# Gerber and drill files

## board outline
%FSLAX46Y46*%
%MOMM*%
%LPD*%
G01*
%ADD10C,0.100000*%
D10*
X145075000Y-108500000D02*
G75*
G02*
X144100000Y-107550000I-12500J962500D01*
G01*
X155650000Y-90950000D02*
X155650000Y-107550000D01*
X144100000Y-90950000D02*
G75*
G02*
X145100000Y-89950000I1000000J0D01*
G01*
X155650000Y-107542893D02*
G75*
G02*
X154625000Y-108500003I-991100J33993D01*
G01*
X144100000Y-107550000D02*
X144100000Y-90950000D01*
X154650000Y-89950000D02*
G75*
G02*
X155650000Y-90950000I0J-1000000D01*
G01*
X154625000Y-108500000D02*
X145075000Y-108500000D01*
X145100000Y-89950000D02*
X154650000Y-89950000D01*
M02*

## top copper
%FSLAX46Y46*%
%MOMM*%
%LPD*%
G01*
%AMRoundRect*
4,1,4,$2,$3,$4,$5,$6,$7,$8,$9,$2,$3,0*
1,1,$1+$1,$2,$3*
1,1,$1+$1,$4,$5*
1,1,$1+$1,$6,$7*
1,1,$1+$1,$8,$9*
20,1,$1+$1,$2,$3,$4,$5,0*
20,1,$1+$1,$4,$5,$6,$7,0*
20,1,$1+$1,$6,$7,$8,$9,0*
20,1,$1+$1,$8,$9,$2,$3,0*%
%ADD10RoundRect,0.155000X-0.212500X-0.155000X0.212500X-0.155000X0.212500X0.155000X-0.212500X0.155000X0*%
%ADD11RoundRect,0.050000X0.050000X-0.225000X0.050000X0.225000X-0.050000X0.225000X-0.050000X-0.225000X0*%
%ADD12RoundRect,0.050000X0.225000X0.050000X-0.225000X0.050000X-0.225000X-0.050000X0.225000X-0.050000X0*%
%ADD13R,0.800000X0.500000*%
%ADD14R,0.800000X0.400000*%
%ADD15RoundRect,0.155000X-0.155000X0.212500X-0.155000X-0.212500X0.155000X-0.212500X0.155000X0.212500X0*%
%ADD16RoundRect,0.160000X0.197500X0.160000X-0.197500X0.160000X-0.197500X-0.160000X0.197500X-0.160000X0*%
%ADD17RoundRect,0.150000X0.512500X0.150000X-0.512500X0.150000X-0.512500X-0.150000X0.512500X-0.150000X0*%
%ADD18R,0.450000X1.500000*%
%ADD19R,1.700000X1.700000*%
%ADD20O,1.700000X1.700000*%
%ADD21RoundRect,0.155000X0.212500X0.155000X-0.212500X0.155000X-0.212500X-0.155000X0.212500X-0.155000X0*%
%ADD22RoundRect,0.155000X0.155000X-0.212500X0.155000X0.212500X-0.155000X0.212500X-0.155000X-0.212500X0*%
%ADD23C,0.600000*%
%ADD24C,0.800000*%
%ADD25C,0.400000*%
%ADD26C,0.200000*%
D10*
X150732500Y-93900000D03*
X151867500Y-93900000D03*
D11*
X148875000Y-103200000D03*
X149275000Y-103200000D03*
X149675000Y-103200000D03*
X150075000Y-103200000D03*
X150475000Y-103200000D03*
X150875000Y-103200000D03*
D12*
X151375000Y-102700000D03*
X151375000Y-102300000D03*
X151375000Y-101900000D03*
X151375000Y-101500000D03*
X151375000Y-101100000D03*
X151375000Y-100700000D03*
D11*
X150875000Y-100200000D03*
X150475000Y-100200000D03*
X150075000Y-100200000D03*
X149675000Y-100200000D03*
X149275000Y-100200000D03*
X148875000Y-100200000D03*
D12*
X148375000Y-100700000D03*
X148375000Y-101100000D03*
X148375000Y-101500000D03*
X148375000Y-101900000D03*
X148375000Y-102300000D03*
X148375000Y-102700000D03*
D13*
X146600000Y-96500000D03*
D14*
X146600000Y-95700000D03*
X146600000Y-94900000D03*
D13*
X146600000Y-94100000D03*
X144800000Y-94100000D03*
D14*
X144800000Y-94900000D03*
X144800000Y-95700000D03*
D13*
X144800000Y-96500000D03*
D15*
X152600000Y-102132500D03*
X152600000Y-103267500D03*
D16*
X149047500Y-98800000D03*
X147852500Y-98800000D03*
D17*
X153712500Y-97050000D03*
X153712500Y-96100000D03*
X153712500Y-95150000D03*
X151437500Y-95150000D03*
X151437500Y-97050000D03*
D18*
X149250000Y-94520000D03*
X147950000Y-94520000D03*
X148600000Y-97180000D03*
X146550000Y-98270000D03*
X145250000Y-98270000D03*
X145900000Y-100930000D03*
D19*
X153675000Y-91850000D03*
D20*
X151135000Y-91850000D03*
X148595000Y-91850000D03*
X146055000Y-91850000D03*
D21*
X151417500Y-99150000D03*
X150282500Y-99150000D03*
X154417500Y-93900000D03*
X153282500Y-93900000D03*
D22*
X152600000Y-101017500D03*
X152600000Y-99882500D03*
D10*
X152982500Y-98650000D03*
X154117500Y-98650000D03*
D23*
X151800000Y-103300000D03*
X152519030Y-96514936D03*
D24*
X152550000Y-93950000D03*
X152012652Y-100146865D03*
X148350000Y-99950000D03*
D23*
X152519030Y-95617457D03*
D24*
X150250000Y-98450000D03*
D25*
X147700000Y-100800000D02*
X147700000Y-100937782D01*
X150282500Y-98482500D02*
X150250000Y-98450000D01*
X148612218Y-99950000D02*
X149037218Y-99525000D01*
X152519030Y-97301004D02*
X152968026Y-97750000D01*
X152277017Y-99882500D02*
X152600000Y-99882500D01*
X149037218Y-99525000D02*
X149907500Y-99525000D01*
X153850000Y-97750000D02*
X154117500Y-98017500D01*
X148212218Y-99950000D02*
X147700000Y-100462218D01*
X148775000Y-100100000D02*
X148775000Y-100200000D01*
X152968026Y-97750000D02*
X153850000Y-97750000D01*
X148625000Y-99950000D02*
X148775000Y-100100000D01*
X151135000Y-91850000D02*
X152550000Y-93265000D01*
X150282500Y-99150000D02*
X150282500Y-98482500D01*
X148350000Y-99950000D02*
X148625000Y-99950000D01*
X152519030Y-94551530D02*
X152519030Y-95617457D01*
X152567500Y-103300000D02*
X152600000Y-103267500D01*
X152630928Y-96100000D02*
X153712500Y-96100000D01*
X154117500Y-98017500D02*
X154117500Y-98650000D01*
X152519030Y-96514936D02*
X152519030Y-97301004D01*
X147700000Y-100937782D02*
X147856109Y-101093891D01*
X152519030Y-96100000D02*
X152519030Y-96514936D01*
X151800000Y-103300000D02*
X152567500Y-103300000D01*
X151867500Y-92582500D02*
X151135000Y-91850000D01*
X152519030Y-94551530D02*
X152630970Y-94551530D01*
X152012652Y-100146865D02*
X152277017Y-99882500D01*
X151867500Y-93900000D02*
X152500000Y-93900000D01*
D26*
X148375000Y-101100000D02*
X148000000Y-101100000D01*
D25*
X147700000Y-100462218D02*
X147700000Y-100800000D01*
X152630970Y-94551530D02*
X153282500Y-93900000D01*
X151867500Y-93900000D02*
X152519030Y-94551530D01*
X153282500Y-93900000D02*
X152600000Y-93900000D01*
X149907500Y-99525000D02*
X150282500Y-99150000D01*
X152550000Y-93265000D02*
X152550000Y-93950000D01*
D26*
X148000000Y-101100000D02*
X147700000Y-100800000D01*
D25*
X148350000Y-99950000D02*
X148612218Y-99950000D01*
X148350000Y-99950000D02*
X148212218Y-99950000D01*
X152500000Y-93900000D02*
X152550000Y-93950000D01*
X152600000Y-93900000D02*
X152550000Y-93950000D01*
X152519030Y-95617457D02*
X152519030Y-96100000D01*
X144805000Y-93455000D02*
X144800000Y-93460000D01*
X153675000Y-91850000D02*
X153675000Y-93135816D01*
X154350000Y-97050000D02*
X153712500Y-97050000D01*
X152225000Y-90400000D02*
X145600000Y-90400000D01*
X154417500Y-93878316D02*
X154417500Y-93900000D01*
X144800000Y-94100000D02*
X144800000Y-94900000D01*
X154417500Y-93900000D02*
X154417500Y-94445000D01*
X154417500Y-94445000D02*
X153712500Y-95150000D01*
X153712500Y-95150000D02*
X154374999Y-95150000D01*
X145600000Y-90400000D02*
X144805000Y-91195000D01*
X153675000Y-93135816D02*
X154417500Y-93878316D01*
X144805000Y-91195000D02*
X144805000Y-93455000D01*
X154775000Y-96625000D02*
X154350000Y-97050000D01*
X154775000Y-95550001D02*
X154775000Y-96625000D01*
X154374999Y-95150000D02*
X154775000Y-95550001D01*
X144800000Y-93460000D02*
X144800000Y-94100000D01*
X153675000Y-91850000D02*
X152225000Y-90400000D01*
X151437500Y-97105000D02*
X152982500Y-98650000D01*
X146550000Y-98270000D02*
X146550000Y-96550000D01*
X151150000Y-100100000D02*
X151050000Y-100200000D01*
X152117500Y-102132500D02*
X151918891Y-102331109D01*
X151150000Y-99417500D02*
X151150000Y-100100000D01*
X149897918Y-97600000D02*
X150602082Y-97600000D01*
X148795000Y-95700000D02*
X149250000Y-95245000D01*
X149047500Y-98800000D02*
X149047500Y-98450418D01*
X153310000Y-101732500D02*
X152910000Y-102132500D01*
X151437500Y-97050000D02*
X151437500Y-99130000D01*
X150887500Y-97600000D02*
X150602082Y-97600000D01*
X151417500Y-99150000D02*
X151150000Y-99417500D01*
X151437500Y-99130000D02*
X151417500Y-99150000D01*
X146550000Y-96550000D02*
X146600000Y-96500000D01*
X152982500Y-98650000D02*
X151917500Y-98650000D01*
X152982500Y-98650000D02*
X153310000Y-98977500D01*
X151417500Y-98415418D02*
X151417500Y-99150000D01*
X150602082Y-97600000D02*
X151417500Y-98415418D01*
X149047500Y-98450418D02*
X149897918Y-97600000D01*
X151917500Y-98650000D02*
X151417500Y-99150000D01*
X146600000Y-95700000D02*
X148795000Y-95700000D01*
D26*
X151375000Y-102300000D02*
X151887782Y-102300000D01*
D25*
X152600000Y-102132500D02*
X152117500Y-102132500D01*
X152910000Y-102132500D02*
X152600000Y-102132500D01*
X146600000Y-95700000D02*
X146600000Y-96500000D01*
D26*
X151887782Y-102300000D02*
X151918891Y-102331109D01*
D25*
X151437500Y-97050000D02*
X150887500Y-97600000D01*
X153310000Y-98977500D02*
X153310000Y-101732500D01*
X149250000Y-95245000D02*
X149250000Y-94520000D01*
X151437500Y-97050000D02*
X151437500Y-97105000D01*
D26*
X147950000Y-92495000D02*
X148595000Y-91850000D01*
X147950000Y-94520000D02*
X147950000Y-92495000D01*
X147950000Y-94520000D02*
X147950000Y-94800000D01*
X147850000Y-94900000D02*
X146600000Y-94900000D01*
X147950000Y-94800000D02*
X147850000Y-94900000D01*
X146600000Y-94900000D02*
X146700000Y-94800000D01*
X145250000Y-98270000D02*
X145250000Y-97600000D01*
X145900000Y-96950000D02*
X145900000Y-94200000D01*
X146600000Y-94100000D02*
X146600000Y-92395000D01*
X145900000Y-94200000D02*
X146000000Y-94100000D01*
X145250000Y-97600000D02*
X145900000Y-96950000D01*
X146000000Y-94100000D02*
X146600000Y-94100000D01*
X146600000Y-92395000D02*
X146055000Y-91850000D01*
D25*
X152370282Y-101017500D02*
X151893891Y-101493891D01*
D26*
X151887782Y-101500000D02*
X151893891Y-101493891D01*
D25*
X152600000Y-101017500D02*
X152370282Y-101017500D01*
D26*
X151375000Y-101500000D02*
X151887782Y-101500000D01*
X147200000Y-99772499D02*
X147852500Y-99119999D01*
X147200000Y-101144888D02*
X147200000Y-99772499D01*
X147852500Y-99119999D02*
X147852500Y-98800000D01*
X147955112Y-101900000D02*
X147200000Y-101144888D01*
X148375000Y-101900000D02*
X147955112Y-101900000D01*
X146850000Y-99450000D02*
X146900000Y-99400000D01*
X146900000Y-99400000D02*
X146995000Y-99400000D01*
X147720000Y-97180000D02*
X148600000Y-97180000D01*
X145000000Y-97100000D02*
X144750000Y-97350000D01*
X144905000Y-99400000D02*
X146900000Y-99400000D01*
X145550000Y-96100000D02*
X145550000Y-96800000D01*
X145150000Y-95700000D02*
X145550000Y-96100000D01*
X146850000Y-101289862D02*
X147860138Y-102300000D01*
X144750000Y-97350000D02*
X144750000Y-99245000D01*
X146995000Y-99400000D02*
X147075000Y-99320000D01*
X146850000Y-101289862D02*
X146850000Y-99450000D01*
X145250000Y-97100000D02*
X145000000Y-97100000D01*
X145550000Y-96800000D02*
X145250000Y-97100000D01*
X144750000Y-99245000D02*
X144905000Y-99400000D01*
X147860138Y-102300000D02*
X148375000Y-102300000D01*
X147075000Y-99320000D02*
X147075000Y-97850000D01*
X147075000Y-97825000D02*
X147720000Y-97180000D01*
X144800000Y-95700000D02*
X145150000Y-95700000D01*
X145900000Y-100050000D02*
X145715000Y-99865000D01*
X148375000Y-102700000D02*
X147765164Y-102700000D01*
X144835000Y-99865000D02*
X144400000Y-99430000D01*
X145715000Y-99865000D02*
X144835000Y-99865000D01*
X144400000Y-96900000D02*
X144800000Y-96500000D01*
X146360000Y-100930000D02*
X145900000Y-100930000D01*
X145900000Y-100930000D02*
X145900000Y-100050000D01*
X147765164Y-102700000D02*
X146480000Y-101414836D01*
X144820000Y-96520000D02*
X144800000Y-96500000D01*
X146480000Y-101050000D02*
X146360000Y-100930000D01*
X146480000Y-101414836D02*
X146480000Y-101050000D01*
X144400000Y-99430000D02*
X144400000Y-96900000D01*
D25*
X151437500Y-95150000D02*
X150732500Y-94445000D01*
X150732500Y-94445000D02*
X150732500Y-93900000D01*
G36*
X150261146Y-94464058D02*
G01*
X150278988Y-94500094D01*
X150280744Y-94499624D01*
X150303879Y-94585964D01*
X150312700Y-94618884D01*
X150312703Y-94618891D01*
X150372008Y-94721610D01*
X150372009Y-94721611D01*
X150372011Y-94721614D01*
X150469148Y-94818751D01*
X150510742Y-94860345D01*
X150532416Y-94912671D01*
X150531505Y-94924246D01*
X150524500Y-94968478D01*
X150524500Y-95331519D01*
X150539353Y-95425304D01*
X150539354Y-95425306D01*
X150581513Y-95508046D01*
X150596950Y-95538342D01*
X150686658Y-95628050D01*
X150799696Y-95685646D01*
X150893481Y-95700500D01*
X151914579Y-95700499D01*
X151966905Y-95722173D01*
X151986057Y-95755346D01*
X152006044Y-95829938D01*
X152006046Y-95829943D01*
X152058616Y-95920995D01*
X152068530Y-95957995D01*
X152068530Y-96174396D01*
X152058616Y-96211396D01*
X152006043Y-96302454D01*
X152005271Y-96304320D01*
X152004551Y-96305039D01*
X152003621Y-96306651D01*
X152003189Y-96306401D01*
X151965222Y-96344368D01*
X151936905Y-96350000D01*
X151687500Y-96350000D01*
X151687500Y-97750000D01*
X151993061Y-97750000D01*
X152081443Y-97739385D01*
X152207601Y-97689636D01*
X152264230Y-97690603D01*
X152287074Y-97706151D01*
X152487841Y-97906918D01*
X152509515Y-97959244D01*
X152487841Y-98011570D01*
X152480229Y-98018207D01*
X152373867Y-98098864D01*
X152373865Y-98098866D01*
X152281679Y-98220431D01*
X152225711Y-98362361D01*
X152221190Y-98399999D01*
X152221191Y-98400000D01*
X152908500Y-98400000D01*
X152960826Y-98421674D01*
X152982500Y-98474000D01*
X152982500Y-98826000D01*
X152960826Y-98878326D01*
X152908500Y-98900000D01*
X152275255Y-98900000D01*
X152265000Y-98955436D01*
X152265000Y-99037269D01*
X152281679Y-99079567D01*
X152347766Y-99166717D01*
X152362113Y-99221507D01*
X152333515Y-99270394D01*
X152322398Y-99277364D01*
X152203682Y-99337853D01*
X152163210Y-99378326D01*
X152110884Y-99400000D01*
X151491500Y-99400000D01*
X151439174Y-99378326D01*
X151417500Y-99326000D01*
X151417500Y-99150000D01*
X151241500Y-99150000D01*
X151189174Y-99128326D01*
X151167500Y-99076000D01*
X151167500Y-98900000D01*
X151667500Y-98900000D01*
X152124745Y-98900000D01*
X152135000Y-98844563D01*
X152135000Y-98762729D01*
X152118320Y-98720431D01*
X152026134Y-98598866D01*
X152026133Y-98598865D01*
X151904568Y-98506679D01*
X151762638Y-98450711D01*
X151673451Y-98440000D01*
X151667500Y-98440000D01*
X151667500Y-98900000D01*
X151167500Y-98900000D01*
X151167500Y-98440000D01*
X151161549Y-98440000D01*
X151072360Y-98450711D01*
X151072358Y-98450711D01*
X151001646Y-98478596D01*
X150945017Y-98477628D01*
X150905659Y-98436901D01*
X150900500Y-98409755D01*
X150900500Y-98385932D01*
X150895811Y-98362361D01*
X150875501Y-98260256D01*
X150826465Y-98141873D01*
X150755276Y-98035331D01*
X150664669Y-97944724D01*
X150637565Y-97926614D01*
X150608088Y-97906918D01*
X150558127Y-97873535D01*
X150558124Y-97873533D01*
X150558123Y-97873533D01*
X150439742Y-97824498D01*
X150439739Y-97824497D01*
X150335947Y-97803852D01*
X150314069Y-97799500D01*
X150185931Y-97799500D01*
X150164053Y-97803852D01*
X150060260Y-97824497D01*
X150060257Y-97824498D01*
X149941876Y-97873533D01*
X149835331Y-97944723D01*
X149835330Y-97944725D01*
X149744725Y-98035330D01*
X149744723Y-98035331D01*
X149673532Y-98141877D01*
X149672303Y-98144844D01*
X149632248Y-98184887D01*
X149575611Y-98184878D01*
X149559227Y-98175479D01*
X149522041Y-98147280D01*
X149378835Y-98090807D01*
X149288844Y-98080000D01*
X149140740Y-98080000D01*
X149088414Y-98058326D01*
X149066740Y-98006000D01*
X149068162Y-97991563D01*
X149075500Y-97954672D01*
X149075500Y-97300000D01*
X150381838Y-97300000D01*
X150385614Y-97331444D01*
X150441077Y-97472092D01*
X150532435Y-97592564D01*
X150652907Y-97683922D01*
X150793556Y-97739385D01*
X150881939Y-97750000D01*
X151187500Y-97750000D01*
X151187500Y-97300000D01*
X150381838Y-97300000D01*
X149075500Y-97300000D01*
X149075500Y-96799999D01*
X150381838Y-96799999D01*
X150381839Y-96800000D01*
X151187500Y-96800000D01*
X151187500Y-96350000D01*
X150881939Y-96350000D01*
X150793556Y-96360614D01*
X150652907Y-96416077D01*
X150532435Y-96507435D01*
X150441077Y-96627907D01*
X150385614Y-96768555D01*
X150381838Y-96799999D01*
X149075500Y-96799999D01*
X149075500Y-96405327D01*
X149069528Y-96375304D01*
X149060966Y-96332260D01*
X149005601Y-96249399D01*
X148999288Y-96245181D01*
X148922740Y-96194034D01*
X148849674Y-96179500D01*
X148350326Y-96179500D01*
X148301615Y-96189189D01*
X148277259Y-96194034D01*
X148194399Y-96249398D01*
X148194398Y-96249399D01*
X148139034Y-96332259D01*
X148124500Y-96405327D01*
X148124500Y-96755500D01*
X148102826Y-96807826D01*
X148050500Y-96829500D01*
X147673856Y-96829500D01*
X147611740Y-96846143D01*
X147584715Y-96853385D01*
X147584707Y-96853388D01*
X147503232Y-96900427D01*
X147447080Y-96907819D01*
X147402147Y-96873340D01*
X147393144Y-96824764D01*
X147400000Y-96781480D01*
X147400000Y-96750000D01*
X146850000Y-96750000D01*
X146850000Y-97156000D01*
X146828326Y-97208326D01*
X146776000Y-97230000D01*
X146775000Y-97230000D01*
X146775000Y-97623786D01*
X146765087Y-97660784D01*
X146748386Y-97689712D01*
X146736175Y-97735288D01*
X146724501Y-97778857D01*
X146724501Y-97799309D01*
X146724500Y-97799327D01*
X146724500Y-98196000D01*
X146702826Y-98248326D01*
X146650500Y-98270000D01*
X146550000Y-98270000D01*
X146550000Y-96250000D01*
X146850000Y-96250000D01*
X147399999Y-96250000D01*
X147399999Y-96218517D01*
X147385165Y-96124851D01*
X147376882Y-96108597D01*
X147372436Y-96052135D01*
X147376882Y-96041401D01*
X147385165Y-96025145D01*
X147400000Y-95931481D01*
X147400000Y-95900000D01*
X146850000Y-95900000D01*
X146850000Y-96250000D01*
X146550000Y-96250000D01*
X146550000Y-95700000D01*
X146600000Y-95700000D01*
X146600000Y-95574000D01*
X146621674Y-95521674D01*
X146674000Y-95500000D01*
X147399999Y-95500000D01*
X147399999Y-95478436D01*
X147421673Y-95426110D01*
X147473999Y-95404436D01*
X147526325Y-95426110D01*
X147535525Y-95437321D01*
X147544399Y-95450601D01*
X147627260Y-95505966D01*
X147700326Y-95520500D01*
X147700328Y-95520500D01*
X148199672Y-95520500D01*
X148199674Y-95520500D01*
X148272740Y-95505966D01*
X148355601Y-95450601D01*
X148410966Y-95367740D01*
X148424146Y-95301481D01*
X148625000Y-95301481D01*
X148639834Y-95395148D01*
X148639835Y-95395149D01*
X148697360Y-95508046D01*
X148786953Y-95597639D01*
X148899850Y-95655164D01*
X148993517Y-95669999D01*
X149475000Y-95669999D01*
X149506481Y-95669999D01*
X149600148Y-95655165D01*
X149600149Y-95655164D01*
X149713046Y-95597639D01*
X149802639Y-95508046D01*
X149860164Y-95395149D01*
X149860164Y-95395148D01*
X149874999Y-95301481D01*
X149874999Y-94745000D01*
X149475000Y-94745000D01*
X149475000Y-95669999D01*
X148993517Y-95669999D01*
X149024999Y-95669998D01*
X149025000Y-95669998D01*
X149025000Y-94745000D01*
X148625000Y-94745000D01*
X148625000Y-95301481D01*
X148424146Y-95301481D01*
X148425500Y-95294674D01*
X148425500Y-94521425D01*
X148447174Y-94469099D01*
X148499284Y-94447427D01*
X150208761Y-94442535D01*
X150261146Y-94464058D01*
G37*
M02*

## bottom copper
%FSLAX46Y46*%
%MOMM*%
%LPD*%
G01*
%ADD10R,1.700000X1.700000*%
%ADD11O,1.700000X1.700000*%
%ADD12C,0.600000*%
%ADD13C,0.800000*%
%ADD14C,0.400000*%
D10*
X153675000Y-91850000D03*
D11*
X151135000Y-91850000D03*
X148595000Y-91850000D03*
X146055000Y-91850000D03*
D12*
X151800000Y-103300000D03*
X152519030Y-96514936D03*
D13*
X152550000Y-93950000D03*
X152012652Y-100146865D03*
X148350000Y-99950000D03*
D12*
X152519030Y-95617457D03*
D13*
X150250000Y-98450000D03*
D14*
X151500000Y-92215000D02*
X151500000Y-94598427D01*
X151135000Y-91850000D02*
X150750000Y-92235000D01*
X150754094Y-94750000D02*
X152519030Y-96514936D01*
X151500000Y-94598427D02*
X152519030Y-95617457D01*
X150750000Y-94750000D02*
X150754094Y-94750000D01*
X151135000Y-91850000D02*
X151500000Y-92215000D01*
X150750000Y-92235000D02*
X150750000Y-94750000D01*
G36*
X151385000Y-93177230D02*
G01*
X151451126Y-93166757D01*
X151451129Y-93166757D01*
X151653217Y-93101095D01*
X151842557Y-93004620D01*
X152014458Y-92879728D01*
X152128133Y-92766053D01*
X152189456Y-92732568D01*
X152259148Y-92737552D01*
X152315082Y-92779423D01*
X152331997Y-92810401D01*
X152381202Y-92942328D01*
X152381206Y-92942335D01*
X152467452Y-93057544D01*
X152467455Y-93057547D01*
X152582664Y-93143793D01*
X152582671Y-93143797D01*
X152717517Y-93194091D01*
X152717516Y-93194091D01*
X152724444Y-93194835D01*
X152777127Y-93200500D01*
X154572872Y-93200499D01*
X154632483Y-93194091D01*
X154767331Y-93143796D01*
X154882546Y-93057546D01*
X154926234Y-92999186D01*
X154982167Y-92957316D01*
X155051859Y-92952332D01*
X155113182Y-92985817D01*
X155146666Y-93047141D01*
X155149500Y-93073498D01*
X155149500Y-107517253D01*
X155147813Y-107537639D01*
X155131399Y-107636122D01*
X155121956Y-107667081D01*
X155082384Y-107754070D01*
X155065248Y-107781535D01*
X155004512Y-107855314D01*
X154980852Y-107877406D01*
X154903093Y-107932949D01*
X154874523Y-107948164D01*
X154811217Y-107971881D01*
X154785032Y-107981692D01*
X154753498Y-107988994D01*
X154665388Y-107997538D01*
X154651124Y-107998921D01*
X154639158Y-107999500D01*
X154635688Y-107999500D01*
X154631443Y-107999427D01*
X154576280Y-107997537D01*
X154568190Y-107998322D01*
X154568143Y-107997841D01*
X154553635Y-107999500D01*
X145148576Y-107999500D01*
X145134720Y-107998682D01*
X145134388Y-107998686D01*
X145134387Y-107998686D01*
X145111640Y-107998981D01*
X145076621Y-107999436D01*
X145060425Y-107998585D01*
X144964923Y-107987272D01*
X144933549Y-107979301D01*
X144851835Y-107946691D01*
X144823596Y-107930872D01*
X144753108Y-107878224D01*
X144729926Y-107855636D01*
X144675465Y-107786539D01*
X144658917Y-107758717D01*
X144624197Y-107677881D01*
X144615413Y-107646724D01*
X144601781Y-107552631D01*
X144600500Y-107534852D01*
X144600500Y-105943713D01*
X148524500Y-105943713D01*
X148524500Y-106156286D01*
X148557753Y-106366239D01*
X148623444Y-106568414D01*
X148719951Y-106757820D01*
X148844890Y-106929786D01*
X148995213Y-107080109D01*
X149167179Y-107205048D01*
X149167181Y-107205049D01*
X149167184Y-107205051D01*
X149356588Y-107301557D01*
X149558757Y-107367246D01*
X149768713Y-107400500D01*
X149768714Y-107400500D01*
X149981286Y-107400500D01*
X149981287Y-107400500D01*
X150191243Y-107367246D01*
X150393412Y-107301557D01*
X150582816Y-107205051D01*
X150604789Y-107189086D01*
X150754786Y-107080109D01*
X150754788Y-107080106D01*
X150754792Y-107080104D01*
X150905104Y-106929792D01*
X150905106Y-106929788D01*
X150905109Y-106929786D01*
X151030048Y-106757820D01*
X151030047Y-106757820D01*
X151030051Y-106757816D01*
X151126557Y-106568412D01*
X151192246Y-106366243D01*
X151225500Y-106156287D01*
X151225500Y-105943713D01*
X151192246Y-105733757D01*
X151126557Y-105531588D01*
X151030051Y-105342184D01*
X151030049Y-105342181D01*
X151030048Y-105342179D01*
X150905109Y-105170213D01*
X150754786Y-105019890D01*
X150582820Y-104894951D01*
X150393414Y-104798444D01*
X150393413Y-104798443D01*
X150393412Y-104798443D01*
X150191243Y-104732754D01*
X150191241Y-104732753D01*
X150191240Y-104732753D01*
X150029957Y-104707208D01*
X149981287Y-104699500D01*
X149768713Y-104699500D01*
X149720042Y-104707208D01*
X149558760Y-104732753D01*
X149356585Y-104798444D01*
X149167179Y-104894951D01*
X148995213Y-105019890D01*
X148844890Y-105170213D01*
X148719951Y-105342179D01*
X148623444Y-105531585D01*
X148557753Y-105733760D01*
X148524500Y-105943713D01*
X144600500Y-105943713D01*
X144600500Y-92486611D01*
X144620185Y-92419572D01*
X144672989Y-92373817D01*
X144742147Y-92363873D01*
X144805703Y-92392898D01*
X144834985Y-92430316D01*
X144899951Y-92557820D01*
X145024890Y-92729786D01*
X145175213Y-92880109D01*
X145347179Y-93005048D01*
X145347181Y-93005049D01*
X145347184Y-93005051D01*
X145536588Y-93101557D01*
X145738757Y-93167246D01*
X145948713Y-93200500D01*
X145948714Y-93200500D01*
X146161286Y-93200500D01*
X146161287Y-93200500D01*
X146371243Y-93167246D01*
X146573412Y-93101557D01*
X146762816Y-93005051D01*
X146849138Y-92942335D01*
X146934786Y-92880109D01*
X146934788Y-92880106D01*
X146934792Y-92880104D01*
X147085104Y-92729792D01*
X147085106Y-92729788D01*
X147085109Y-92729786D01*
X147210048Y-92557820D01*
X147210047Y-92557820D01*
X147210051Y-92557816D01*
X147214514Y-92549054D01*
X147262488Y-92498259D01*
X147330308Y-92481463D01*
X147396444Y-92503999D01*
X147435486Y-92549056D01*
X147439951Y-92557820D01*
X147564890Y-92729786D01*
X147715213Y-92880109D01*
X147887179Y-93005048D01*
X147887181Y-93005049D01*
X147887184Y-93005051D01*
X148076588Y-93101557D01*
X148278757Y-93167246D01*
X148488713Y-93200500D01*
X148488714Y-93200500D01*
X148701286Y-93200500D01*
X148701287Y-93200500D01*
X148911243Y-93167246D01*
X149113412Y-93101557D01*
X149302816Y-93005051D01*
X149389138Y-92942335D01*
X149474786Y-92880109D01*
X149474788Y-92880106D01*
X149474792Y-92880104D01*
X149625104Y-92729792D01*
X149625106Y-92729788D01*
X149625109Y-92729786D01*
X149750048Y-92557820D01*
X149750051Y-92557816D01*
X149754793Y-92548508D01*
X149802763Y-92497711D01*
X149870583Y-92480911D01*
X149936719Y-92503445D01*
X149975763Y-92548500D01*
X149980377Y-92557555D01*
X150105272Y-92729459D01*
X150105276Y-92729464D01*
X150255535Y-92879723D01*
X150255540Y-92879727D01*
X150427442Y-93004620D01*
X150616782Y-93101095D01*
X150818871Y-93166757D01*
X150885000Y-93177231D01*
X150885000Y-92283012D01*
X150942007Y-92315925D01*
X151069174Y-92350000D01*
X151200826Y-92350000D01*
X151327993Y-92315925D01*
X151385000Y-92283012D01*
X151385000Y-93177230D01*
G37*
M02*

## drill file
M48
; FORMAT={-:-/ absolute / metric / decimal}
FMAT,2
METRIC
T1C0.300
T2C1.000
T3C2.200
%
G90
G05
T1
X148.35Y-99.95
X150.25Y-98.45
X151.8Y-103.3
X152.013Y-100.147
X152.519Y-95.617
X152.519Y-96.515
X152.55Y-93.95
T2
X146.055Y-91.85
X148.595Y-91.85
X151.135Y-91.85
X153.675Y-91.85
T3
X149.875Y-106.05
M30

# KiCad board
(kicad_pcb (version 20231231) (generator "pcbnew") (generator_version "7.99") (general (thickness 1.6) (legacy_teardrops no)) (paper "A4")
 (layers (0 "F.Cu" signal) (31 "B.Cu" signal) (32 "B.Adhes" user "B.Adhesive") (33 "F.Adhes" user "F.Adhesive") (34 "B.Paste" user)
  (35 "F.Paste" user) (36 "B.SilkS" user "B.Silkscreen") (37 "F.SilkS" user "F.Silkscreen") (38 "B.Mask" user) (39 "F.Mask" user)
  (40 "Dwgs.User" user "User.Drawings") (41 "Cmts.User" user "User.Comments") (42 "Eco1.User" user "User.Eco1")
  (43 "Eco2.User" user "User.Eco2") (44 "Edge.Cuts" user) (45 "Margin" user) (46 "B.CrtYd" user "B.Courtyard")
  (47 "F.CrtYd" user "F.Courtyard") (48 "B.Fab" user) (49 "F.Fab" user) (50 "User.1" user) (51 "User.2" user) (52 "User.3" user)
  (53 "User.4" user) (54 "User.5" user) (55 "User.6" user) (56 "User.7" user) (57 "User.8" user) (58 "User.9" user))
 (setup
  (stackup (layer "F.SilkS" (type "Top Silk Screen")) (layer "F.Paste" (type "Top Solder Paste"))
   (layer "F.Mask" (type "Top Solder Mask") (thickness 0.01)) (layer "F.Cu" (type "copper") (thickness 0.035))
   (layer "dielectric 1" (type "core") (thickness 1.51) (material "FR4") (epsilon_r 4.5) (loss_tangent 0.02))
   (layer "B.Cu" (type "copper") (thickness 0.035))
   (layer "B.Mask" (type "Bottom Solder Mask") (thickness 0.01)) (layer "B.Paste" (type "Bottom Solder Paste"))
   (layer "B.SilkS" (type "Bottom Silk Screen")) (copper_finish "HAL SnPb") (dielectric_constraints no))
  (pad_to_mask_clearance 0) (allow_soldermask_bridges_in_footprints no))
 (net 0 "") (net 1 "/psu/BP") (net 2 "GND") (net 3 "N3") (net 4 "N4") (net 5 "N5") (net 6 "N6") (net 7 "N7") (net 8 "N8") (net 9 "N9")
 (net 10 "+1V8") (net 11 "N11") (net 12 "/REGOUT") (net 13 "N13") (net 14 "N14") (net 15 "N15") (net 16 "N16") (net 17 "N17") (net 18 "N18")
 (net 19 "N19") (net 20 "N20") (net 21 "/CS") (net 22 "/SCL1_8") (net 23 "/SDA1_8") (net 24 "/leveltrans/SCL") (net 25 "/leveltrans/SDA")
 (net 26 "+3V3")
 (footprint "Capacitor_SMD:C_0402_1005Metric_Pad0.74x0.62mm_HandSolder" (layer "F.Cu") (at 151.3 93.9)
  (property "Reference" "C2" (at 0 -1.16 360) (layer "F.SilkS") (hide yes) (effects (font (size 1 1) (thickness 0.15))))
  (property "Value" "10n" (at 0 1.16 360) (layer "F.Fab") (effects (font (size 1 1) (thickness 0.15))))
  (pad "1" smd roundrect (at -0.5675 0) (size 0.735 0.62) (layers "F.Cu" "F.Paste" "F.Mask") (roundrect_rratio 0.25) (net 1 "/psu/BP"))
  (pad "2" smd roundrect (at 0.5675 0) (size 0.735 0.62) (layers "F.Cu" "F.Paste" "F.Mask") (roundrect_rratio 0.25) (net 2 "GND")))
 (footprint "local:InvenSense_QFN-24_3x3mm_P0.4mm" (layer "F.Cu") (at 149.875 101.7 90)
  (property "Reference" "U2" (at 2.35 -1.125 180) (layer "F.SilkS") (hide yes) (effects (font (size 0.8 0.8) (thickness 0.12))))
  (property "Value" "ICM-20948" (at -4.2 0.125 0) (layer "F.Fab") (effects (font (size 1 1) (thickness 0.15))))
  (pad "1" smd roundrect (at -1.5 -1 90) (size 0.55 0.2) (layers "F.Cu" "F.Paste" "F.Mask") (roundrect_rratio 0.25) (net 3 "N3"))
  (pad "2" smd roundrect (at -1.5 -0.6 90) (size 0.55 0.2) (layers "F.Cu" "F.Paste" "F.Mask") (roundrect_rratio 0.25) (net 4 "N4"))
  (pad "3" smd roundrect (at -1.5 -0.2 90) (size 0.55 0.2) (layers "F.Cu" "F.Paste" "F.Mask") (roundrect_rratio 0.25) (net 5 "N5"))
  (pad "4" smd roundrect (at -1.5 0.2 90) (size 0.55 0.2) (layers "F.Cu" "F.Paste" "F.Mask") (roundrect_rratio 0.25) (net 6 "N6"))
  (pad "5" smd roundrect (at -1.5 0.6 90) (size 0.55 0.2) (layers "F.Cu" "F.Paste" "F.Mask") (roundrect_rratio 0.25) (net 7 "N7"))
  (pad "6" smd roundrect (at -1.5 1 90) (size 0.55 0.2) (layers "F.Cu" "F.Paste" "F.Mask") (roundrect_rratio 0.25) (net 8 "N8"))
  (pad "7" smd roundrect (at -1 1.5 180) (size 0.55 0.2) (layers "F.Cu" "F.Paste" "F.Mask") (roundrect_rratio 0.25) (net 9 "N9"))
  (pad "8" smd roundrect (at -0.6 1.5 180) (size 0.55 0.2) (layers "F.Cu" "F.Paste" "F.Mask") (roundrect_rratio 0.25) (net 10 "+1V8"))
  (pad "9" smd roundrect (at -0.2 1.5 180) (size 0.55 0.2) (layers "F.Cu" "F.Paste" "F.Mask") (roundrect_rratio 0.25) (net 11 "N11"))
  (pad "10" smd roundrect (at 0.2 1.5 180) (size 0.55 0.2) (layers "F.Cu" "F.Paste" "F.Mask") (roundrect_rratio 0.25) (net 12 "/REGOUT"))
  (pad "11" smd roundrect (at 0.6 1.5 180) (size 0.55 0.2) (layers "F.Cu" "F.Paste" "F.Mask") (roundrect_rratio 0.25) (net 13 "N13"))
  (pad "12" smd roundrect (at 1 1.5 180) (size 0.55 0.2) (layers "F.Cu" "F.Paste" "F.Mask") (roundrect_rratio 0.25) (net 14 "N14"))
  (pad "13" smd roundrect (at 1.5 1 90) (size 0.55 0.2) (layers "F.Cu" "F.Paste" "F.Mask") (roundrect_rratio 0.25) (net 10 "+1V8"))
  (pad "14" smd roundrect (at 1.5 0.6 90) (size 0.55 0.2) (layers "F.Cu" "F.Paste" "F.Mask") (roundrect_rratio 0.25) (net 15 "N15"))
  (pad "15" smd roundrect (at 1.5 0.2 90) (size 0.55 0.2) (layers "F.Cu" "F.Paste" "F.Mask") (roundrect_rratio 0.25) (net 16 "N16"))
  (pad "16" smd roundrect (at 1.5 -0.2 90) (size 0.55 0.2) (layers "F.Cu" "F.Paste" "F.Mask") (roundrect_rratio 0.25) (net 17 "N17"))
  (pad "17" smd roundrect (at 1.5 -0.6 90) (size 0.55 0.2) (layers "F.Cu" "F.Paste" "F.Mask") (roundrect_rratio 0.25) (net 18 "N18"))
  (pad "18" smd roundrect (at 1.5 -1 90) (size 0.55 0.2) (layers "F.Cu" "F.Paste" "F.Mask") (roundrect_rratio 0.25) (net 2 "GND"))
  (pad "19" smd roundrect (at 1 -1.5 180) (size 0.55 0.2) (layers "F.Cu" "F.Paste" "F.Mask") (roundrect_rratio 0.25) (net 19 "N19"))
  (pad "20" smd roundrect (at 0.6 -1.5 180) (size 0.55 0.2) (layers "F.Cu" "F.Paste" "F.Mask") (roundrect_rratio 0.25) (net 2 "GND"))
  (pad "21" smd roundrect (at 0.2 -1.5 180) (size 0.55 0.2) (layers "F.Cu" "F.Paste" "F.Mask") (roundrect_rratio 0.25) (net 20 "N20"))
  (pad "22" smd roundrect (at -0.2 -1.5 180) (size 0.55 0.2) (layers "F.Cu" "F.Paste" "F.Mask") (roundrect_rratio 0.25) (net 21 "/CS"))
  (pad "23" smd roundrect (at -0.6 -1.5 180) (size 0.55 0.2) (layers "F.Cu" "F.Paste" "F.Mask") (roundrect_rratio 0.25) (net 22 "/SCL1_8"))
  (pad "24" smd roundrect (at -1 -1.5 180) (size 0.55 0.2) (layers "F.Cu" "F.Paste" "F.Mask") (roundrect_rratio 0.25) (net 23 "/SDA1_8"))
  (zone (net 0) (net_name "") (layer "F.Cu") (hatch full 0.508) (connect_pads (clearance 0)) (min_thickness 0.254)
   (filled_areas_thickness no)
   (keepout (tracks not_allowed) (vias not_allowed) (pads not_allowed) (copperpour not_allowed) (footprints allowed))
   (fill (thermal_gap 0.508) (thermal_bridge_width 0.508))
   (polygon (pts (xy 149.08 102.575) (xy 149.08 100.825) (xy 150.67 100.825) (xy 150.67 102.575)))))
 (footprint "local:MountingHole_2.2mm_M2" (layer "F.Cu") (at 149.875 106.05)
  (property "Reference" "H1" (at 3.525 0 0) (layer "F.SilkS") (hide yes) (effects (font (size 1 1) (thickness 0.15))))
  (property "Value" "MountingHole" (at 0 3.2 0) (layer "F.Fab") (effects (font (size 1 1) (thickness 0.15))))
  (pad "" np_thru_hole circle (at 0 0) (size 2.2 2.2) (drill 2.2) (layers "*.Cu" "*.Mask")))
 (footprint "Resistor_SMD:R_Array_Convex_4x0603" (layer "F.Cu") (at 145.7 95.3 180)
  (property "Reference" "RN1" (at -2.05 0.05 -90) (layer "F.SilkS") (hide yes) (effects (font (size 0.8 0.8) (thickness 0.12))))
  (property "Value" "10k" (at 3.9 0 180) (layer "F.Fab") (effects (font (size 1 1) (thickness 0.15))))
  (pad "1" smd rect (at -0.9 -1.2 180) (size 0.8 0.5) (layers "F.Cu" "F.Paste" "F.Mask") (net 10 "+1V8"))
  (pad "2" smd rect (at -0.9 -0.4 180) (size 0.8 0.4) (layers "F.Cu" "F.Paste" "F.Mask") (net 10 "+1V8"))
  (pad "3" smd rect (at -0.9 0.4 180) (size 0.8 0.4) (layers "F.Cu" "F.Paste" "F.Mask") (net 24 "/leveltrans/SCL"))
  (pad "4" smd rect (at -0.9 1.2 180) (size 0.8 0.5) (layers "F.Cu" "F.Paste" "F.Mask") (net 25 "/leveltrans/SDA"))
  (pad "5" smd rect (at 0.9 1.2 180) (size 0.8 0.5) (layers "F.Cu" "F.Paste" "F.Mask") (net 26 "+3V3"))
  (pad "6" smd rect (at 0.9 0.4 180) (size 0.8 0.4) (layers "F.Cu" "F.Paste" "F.Mask") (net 26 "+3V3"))
  (pad "7" smd rect (at 0.9 -0.4 180) (size 0.8 0.4) (layers "F.Cu" "F.Paste" "F.Mask") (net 22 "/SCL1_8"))
  (pad "8" smd rect (at 0.9 -1.2 180) (size 0.8 0.5) (layers "F.Cu" "F.Paste" "F.Mask") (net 23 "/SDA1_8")))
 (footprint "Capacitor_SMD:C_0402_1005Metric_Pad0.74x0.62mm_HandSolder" (layer "F.Cu") (at 152.6 102.7 -90)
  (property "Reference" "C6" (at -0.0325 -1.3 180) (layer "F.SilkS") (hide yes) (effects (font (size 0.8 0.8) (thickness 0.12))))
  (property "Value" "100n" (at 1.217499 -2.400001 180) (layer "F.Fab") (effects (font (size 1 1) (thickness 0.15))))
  (pad "1" smd roundrect (at -0.5675 0 270) (size 0.735 0.62) (layers "F.Cu" "F.Paste" "F.Mask") (roundrect_rratio 0.25) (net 10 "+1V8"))
  (pad "2" smd roundrect (at 0.5675 0 270) (size 0.735 0.62) (layers "F.Cu" "F.Paste" "F.Mask") (roundrect_rratio 0.25) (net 2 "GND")))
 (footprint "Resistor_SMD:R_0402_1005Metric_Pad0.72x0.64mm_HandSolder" (layer "F.Cu") (at 148.45 98.8 180)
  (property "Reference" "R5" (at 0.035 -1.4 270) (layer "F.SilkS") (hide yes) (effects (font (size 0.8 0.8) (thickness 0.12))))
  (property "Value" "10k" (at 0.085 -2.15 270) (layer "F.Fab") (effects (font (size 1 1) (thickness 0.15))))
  (pad "1" smd roundrect (at -0.5975 0 180) (size 0.715 0.64) (layers "F.Cu" "F.Paste" "F.Mask") (roundrect_rratio 0.25) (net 10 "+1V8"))
  (pad "2" smd roundrect (at 0.5975 0 180) (size 0.715 0.64) (layers "F.Cu" "F.Paste" "F.Mask") (roundrect_rratio 0.25) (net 21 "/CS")))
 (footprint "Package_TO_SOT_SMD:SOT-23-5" (layer "F.Cu") (at 152.575 96.1 180)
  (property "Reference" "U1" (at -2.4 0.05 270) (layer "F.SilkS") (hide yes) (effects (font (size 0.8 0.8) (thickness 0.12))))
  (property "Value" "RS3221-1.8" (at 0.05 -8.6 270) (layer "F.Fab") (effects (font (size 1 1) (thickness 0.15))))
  (pad "1" smd roundrect (at -1.1375 -0.95 180) (size 1.325 0.6) (layers "F.Cu" "F.Paste" "F.Mask") (roundrect_rratio 0.25) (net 26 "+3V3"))
  (pad "2" smd roundrect (at -1.1375 0 180) (size 1.325 0.6) (layers "F.Cu" "F.Paste" "F.Mask") (roundrect_rratio 0.25) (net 2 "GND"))
  (pad "3" smd roundrect (at -1.1375 0.95 180) (size 1.325 0.6) (layers "F.Cu" "F.Paste" "F.Mask") (roundrect_rratio 0.25) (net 26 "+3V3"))
  (pad "4" smd roundrect (at 1.1375 0.95 180) (size 1.325 0.6) (layers "F.Cu" "F.Paste" "F.Mask") (roundrect_rratio 0.25) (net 1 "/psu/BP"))
  (pad "5" smd roundrect (at 1.1375 -0.95 180) (size 1.325 0.6) (layers "F.Cu" "F.Paste" "F.Mask") (roundrect_rratio 0.25) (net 10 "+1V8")))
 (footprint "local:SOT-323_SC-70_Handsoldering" (layer "F.Cu") (at 148.6 95.85 -90)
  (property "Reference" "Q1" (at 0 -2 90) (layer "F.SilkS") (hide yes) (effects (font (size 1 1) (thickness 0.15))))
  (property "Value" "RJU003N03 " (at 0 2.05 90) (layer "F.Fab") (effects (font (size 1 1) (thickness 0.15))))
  (pad "1" smd rect (at -1.33 -0.65 180) (size 0.45 1.5) (layers "F.Cu" "F.Paste" "F.Mask") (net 10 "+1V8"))
  (pad "2" smd rect (at -1.33 0.65 180) (size 0.45 1.5) (layers "F.Cu" "F.Paste" "F.Mask") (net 24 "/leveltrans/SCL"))
  (pad "3" smd rect (at 1.33 0 180) (size 0.45 1.5) (layers "F.Cu" "F.Paste" "F.Mask") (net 22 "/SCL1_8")))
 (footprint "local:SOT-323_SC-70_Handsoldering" (layer "F.Cu") (at 145.9 99.6 -90)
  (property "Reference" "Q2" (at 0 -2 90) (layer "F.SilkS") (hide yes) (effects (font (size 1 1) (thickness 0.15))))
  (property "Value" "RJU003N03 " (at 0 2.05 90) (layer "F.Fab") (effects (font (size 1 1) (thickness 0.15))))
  (pad "1" smd rect (at -1.33 -0.65 180) (size 0.45 1.5) (layers "F.Cu" "F.Paste" "F.Mask") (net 10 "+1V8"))
  (pad "2" smd rect (at -1.33 0.65 180) (size 0.45 1.5) (layers "F.Cu" "F.Paste" "F.Mask") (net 25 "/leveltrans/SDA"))
  (pad "3" smd rect (at 1.33 0 180) (size 0.45 1.5) (layers "F.Cu" "F.Paste" "F.Mask") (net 23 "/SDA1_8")))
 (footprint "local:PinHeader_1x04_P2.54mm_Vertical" (layer "F.Cu") (at 153.675 91.85 -90)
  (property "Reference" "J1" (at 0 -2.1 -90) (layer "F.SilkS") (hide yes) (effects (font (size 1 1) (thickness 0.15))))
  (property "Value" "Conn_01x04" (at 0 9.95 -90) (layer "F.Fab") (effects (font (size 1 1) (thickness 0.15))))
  (pad "1" thru_hole rect (at 0 0 270) (size 1.7 1.7) (drill 1) (layers "*.Cu" "*.Mask") (remove_unused_layers no) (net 26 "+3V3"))
  (pad "2" thru_hole oval (at 0 2.54 270) (size 1.7 1.7) (drill 1) (layers "*.Cu" "*.Mask") (remove_unused_layers no) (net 2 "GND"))
  (pad "3" thru_hole oval (at 0 5.08 270) (size 1.7 1.7) (drill 1) (layers "*.Cu" "*.Mask") (remove_unused_layers no)
   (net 24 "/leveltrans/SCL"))
  (pad "4" thru_hole oval (at 0 7.62 270) (size 1.7 1.7) (drill 1) (layers "*.Cu" "*.Mask") (remove_unused_layers no)
   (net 25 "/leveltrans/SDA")))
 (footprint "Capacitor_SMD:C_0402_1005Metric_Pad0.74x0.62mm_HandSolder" (layer "F.Cu") (at 150.85 99.15 180)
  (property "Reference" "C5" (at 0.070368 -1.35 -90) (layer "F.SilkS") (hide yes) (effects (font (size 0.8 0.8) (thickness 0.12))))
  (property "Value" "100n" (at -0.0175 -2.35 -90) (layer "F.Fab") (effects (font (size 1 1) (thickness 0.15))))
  (pad "1" smd roundrect (at -0.5675 0 180) (size 0.735 0.62) (layers "F.Cu" "F.Paste" "F.Mask") (roundrect_rratio 0.25) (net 10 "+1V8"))
  (pad "2" smd roundrect (at 0.5675 0 180) (size 0.735 0.62) (layers "F.Cu" "F.Paste" "F.Mask") (roundrect_rratio 0.25) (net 2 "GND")))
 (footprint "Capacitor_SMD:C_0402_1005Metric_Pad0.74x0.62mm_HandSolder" (layer "F.Cu") (at 153.85 93.9 180)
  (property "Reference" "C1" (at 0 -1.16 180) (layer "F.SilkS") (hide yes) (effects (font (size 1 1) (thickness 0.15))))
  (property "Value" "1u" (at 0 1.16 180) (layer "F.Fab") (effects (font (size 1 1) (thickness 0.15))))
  (pad "1" smd roundrect (at -0.5675 0 180) (size 0.735 0.62) (layers "F.Cu" "F.Paste" "F.Mask") (roundrect_rratio 0.25) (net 26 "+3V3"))
  (pad "2" smd roundrect (at 0.5675 0 180) (size 0.735 0.62) (layers "F.Cu" "F.Paste" "F.Mask") (roundrect_rratio 0.25) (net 2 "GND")))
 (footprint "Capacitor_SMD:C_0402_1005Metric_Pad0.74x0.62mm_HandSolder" (layer "F.Cu") (at 152.6 100.45 90)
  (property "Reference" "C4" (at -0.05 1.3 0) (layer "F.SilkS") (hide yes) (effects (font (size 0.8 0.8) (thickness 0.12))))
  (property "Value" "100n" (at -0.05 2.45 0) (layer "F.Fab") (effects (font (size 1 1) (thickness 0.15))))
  (pad "1" smd roundrect (at -0.5675 0 90) (size 0.735 0.62) (layers "F.Cu" "F.Paste" "F.Mask") (roundrect_rratio 0.25) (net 12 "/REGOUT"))
  (pad "2" smd roundrect (at 0.5675 0 90) (size 0.735 0.62) (layers "F.Cu" "F.Paste" "F.Mask") (roundrect_rratio 0.25) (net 2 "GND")))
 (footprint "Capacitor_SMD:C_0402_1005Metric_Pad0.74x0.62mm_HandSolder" (layer "F.Cu") (at 153.55 98.65)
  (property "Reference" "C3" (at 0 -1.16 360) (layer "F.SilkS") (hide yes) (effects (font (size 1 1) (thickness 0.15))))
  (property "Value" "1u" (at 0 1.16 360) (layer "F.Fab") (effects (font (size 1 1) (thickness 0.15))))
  (pad "1" smd roundrect (at -0.5675 0) (size 0.735 0.62) (layers "F.Cu" "F.Paste" "F.Mask") (roundrect_rratio 0.25) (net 10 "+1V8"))
  (pad "2" smd roundrect (at 0.5675 0) (size 0.735 0.62) (layers "F.Cu" "F.Paste" "F.Mask") (roundrect_rratio 0.25) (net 2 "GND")))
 (gr_arc (start 145.075 108.5) (mid 144.390748 108.226929) (end 144.1 107.55) (stroke (width 0.1) (type default)) (layer "Edge.Cuts"))
 (gr_line (start 155.65 90.95) (end 155.65 107.55) (stroke (width 0.1) (type default)) (layer "Edge.Cuts"))
 (gr_arc (start 144.1 90.95) (mid 144.392893 90.242893) (end 145.1 89.95) (stroke (width 0.1) (type default)) (layer "Edge.Cuts"))
 (gr_arc (start 155.65 107.542893) (mid 155.335723 108.23373) (end 154.625 108.5) (stroke (width 0.1) (type default)) (layer "Edge.Cuts"))
 (gr_line (start 144.1 107.55) (end 144.1 90.95) (stroke (width 0.1) (type default)) (layer "Edge.Cuts"))
 (gr_arc (start 154.65 89.95) (mid 155.357107 90.242893) (end 155.65 90.95) (stroke (width 0.1) (type default)) (layer "Edge.Cuts"))
 (gr_line (start 154.625 108.5) (end 145.075 108.5) (stroke (width 0.1) (type default)) (layer "Edge.Cuts"))
 (gr_line (start 145.1 89.95) (end 154.65 89.95) (stroke (width 0.1) (type default)) (layer "Edge.Cuts"))
 (segment (start 147.7 100.8) (end 147.7 100.937782) (width 0.4) (layer "F.Cu") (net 2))
 (segment (start 150.2825 98.4825) (end 150.25 98.45) (width 0.4) (layer "F.Cu") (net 2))
 (segment (start 148.612218 99.95) (end 149.037218 99.525) (width 0.4) (layer "F.Cu") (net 2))
 (segment (start 152.51903 97.301004) (end 152.968026 97.75) (width 0.4) (layer "F.Cu") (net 2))
 (segment (start 152.277017 99.8825) (end 152.6 99.8825) (width 0.4) (layer "F.Cu") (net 2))
 (segment (start 149.037218 99.525) (end 149.9075 99.525) (width 0.4) (layer "F.Cu") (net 2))
 (segment (start 153.85 97.75) (end 154.1175 98.0175) (width 0.4) (layer "F.Cu") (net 2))
 (segment (start 148.212218 99.95) (end 147.7 100.462218) (width 0.4) (layer "F.Cu") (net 2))
 (segment (start 148.775 100.1) (end 148.775 100.2) (width 0.4) (layer "F.Cu") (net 2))
 (segment (start 152.968026 97.75) (end 153.85 97.75) (width 0.4) (layer "F.Cu") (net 2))
 (segment (start 148.625 99.95) (end 148.775 100.1) (width 0.4) (layer "F.Cu") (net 2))
 (segment (start 151.135 91.85) (end 152.55 93.265) (width 0.4) (layer "F.Cu") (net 2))
 (segment (start 150.2825 99.15) (end 150.2825 98.4825) (width 0.4) (layer "F.Cu") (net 2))
 (segment (start 148.35 99.95) (end 148.625 99.95) (width 0.4) (layer "F.Cu") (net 2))
 (segment (start 152.51903 94.55153) (end 152.51903 95.617457) (width 0.4) (layer "F.Cu") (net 2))
 (segment (start 152.5675 103.3) (end 152.6 103.2675) (width 0.4) (layer "F.Cu") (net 2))
 (segment (start 152.630928 96.1) (end 153.7125 96.1) (width 0.4) (layer "F.Cu") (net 2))
 (segment (start 154.1175 98.0175) (end 154.1175 98.65) (width 0.4) (layer "F.Cu") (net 2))
 (segment (start 152.51903 96.514936) (end 152.51903 97.301004) (width 0.4) (layer "F.Cu") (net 2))
 (segment (start 147.7 100.937782) (end 147.856109 101.093891) (width 0.4) (layer "F.Cu") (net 2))
 (segment (start 152.51903 96.1) (end 152.51903 96.514936) (width 0.4) (layer "F.Cu") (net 2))
 (segment (start 151.8 103.3) (end 152.5675 103.3) (width 0.4) (layer "F.Cu") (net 2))
 (segment (start 151.8675 92.5825) (end 151.135 91.85) (width 0.4) (layer "F.Cu") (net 2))
 (segment (start 152.51903 94.55153) (end 152.63097 94.55153) (width 0.4) (layer "F.Cu") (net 2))
 (segment (start 152.012652 100.146865) (end 152.277017 99.8825) (width 0.4) (layer "F.Cu") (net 2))
 (segment (start 151.8675 93.9) (end 152.5 93.9) (width 0.4) (layer "F.Cu") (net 2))
 (segment (start 148.375 101.1) (end 148 101.1) (width 0.2) (layer "F.Cu") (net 2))
 (segment (start 147.7 100.462218) (end 147.7 100.8) (width 0.4) (layer "F.Cu") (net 2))
 (segment (start 152.63097 94.55153) (end 153.2825 93.9) (width 0.4) (layer "F.Cu") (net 2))
 (segment (start 151.8675 93.9) (end 152.51903 94.55153) (width 0.4) (layer "F.Cu") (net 2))
 (segment (start 153.2825 93.9) (end 152.6 93.9) (width 0.4) (layer "F.Cu") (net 2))
 (segment (start 149.9075 99.525) (end 150.2825 99.15) (width 0.4) (layer "F.Cu") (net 2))
 (segment (start 152.55 93.265) (end 152.55 93.95) (width 0.4) (layer "F.Cu") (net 2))
 (segment (start 148 101.1) (end 147.7 100.8) (width 0.2) (layer "F.Cu") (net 2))
 (segment (start 148.35 99.95) (end 148.612218 99.95) (width 0.4) (layer "F.Cu") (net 2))
 (segment (start 148.35 99.95) (end 148.212218 99.95) (width 0.4) (layer "F.Cu") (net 2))
 (segment (start 152.5 93.9) (end 152.55 93.95) (width 0.4) (layer "F.Cu") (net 2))
 (segment (start 152.6 93.9) (end 152.55 93.95) (width 0.4) (layer "F.Cu") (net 2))
 (segment (start 152.51903 95.617457) (end 152.51903 96.1) (width 0.4) (layer "F.Cu") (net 2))
 (via (at 151.8 103.3) (size 0.6) (drill 0.3) (layers "F.Cu" "B.Cu") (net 2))
 (via (at 152.51903 96.514936) (size 0.6) (drill 0.3) (layers "F.Cu" "B.Cu") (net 2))
 (via (at 152.55 93.95) (size 0.8) (drill 0.3) (layers "F.Cu" "B.Cu") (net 2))
 (via (at 152.012652 100.146865) (size 0.8) (drill 0.3) (layers "F.Cu" "B.Cu") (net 2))
 (via (at 148.35 99.95) (size 0.8) (drill 0.3) (layers "F.Cu" "B.Cu") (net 2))
 (via (at 152.51903 95.617457) (size 0.6) (drill 0.3) (layers "F.Cu" "B.Cu") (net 2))
 (via (at 150.25 98.45) (size 0.8) (drill 0.3) (layers "F.Cu" "B.Cu") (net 2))
 (segment (start 151.5 92.215) (end 151.5 94.598427) (width 0.4) (layer "B.Cu") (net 2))
 (segment (start 151.135 91.85) (end 150.75 92.235) (width 0.4) (layer "B.Cu") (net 2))
 (segment (start 150.754094 94.75) (end 152.51903 96.514936) (width 0.4) (layer "B.Cu") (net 2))
 (segment (start 151.5 94.598427) (end 152.51903 95.617457) (width 0.4) (layer "B.Cu") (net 2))
 (segment (start 150.75 94.75) (end 150.754094 94.75) (width 0.4) (layer "B.Cu") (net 2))
 (segment (start 151.135 91.85) (end 151.5 92.215) (width 0.4) (layer "B.Cu") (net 2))
 (segment (start 150.75 92.235) (end 150.75 94.75) (width 0.4) (layer "B.Cu") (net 2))
 (segment (start 144.805 93.455) (end 144.8 93.46) (width 0.4) (layer "F.Cu") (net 26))
 (segment (start 153.675 91.85) (end 153.675 93.135816) (width 0.4) (layer "F.Cu") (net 26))
 (segment (start 154.35 97.05) (end 153.7125 97.05) (width 0.4) (layer "F.Cu") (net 26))
 (segment (start 152.225 90.4) (end 145.6 90.4) (width 0.4) (layer "F.Cu") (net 26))
 (segment (start 154.4175 93.878316) (end 154.4175 93.9) (width 0.4) (layer "F.Cu") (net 26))
 (segment (start 144.8 94.1) (end 144.8 94.9) (width 0.4) (layer "F.Cu") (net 26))
 (segment (start 154.4175 93.9) (end 154.4175 94.445) (width 0.4) (layer "F.Cu") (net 26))
 (segment (start 154.4175 94.445) (end 153.7125 95.15) (width 0.4) (layer "F.Cu") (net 26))
 (segment (start 153.7125 95.15) (end 154.374999 95.15) (width 0.4) (layer "F.Cu") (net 26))
 (segment (start 145.6 90.4) (end 144.805 91.195) (width 0.4) (layer "F.Cu") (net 26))
 (segment (start 153.675 93.135816) (end 154.4175 93.878316) (width 0.4) (layer "F.Cu") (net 26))
 (segment (start 144.805 91.195) (end 144.805 93.455) (width 0.4) (layer "F.Cu") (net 26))
 (segment (start 154.775 96.625) (end 154.35 97.05) (width 0.4) (layer "F.Cu") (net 26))
 (segment (start 154.775 95.550001) (end 154.775 96.625) (width 0.4) (layer "F.Cu") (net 26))
 (segment (start 154.374999 95.15) (end 154.775 95.550001) (width 0.4) (layer "F.Cu") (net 26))
 (segment (start 144.8 93.46) (end 144.8 94.1) (width 0.4) (layer "F.Cu") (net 26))
 (segment (start 153.675 91.85) (end 152.225 90.4) (width 0.4) (layer "F.Cu") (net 26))
 (segment (start 151.4375 97.105) (end 152.9825 98.65) (width 0.4) (layer "F.Cu") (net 10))
 (segment (start 146.55 98.27) (end 146.55 96.55) (width 0.4) (layer "F.Cu") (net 10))
 (segment (start 151.15 100.1) (end 151.05 100.2) (width 0.4) (layer "F.Cu") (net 10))
 (segment (start 152.1175 102.1325) (end 151.918891 102.331109) (width 0.4) (layer "F.Cu") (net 10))
 (segment (start 151.15 99.4175) (end 151.15 100.1) (width 0.4) (layer "F.Cu") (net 10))
 (segment (start 149.897918 97.6) (end 150.602082 97.6) (width 0.4) (layer "F.Cu") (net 10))
 (segment (start 148.795 95.7) (end 149.25 95.245) (width 0.4) (layer "F.Cu") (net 10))
 (segment (start 149.0475 98.8) (end 149.0475 98.450418) (width 0.4) (layer "F.Cu") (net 10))
 (segment (start 153.31 101.7325) (end 152.91 102.1325) (width 0.4) (layer "F.Cu") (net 10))
 (segment (start 151.4375 97.05) (end 151.4375 99.13) (width 0.4) (layer "F.Cu") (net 10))
 (segment (start 150.8875 97.6) (end 150.602082 97.6) (width 0.4) (layer "F.Cu") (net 10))
 (segment (start 151.4175 99.15) (end 151.15 99.4175) (width 0.4) (layer "F.Cu") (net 10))
 (segment (start 151.4375 99.13) (end 151.4175 99.15) (width 0.4) (layer "F.Cu") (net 10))
 (segment (start 146.55 96.55) (end 146.6 96.5) (width 0.4) (layer "F.Cu") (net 10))
 (segment (start 152.9825 98.65) (end 151.9175 98.65) (width 0.4) (layer "F.Cu") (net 10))
 (segment (start 152.9825 98.65) (end 153.31 98.9775) (width 0.4) (layer "F.Cu") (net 10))
 (segment (start 151.4175 98.415418) (end 151.4175 99.15) (width 0.4) (layer "F.Cu") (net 10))
 (segment (start 150.602082 97.6) (end 151.4175 98.415418) (width 0.4) (layer "F.Cu") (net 10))
 (segment (start 149.0475 98.450418) (end 149.897918 97.6) (width 0.4) (layer "F.Cu") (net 10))
 (segment (start 151.9175 98.65) (end 151.4175 99.15) (width 0.4) (layer "F.Cu") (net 10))
 (segment (start 146.6 95.7) (end 148.795 95.7) (width 0.4) (layer "F.Cu") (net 10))
 (segment (start 151.375 102.3) (end 151.887782 102.3) (width 0.2) (layer "F.Cu") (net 10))
 (segment (start 152.6 102.1325) (end 152.1175 102.1325) (width 0.4) (layer "F.Cu") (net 10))
 (segment (start 152.91 102.1325) (end 152.6 102.1325) (width 0.4) (layer "F.Cu") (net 10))
 (segment (start 146.6 95.7) (end 146.6 96.5) (width 0.4) (layer "F.Cu") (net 10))
 (segment (start 151.887782 102.3) (end 151.918891 102.331109) (width 0.2) (layer "F.Cu") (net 10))
 (segment (start 151.4375 97.05) (end 150.8875 97.6) (width 0.4) (layer "F.Cu") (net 10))
 (segment (start 153.31 98.9775) (end 153.31 101.7325) (width 0.4) (layer "F.Cu") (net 10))
 (segment (start 149.25 95.245) (end 149.25 94.52) (width 0.4) (layer "F.Cu") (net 10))
 (segment (start 151.4375 97.05) (end 151.4375 97.105) (width 0.4) (layer "F.Cu") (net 10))
 (segment (start 147.95 92.495) (end 148.595 91.85) (width 0.2) (layer "F.Cu") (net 24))
 (segment (start 147.95 94.52) (end 147.95 92.495) (width 0.2) (layer "F.Cu") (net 24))
 (segment (start 147.95 94.52) (end 147.95 94.8) (width 0.2) (layer "F.Cu") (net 24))
 (segment (start 147.85 94.9) (end 146.6 94.9) (width 0.2) (layer "F.Cu") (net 24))
 (segment (start 147.95 94.8) (end 147.85 94.9) (width 0.2) (layer "F.Cu") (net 24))
 (segment (start 146.6 94.9) (end 146.7 94.8) (width 0.2) (layer "F.Cu") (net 24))
 (segment (start 145.25 98.27) (end 145.25 97.6) (width 0.2) (layer "F.Cu") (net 25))
 (segment (start 145.9 96.95) (end 145.9 94.2) (width 0.2) (layer "F.Cu") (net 25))
 (segment (start 146.6 94.1) (end 146.6 92.395) (width 0.2) (layer "F.Cu") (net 25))
 (segment (start 145.9 94.2) (end 146 94.1) (width 0.2) (layer "F.Cu") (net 25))
 (segment (start 145.25 97.6) (end 145.9 96.95) (width 0.2) (layer "F.Cu") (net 25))
 (segment (start 146 94.1) (end 146.6 94.1) (width 0.2) (layer "F.Cu") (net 25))
 (segment (start 146.6 92.395) (end 146.055 91.85) (width 0.2) (layer "F.Cu") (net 25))
 (segment (start 152.370282 101.0175) (end 151.893891 101.493891) (width 0.4) (layer "F.Cu") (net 12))
 (segment (start 151.887782 101.5) (end 151.893891 101.493891) (width 0.2) (layer "F.Cu") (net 12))
 (segment (start 152.6 101.0175) (end 152.370282 101.0175) (width 0.4) (layer "F.Cu") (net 12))
 (segment (start 151.375 101.5) (end 151.887782 101.5) (width 0.2) (layer "F.Cu") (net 12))
 (segment (start 147.2 99.772499) (end 147.8525 99.119999) (width 0.2) (layer "F.Cu") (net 21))
 (segment (start 147.2 101.144888) (end 147.2 99.772499) (width 0.2) (layer "F.Cu") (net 21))
 (segment (start 147.8525 99.119999) (end 147.8525 98.8) (width 0.2) (layer "F.Cu") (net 21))
 (segment (start 147.955112 101.9) (end 147.2 101.144888) (width 0.2) (layer "F.Cu") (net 21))
 (segment (start 148.375 101.9) (end 147.955112 101.9) (width 0.2) (layer "F.Cu") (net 21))
 (segment (start 146.85 99.45) (end 146.9 99.4) (width 0.2) (layer "F.Cu") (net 22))
 (segment (start 146.9 99.4) (end 146.995 99.4) (width 0.2) (layer "F.Cu") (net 22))
 (segment (start 147.72 97.18) (end 148.6 97.18) (width 0.2) (layer "F.Cu") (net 22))
 (segment (start 145 97.1) (end 144.75 97.35) (width 0.2) (layer "F.Cu") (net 22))
 (segment (start 144.905 99.4) (end 146.9 99.4) (width 0.2) (layer "F.Cu") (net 22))
 (segment (start 145.55 96.1) (end 145.55 96.8) (width 0.2) (layer "F.Cu") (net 22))
 (segment (start 145.15 95.7) (end 145.55 96.1) (width 0.2) (layer "F.Cu") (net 22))
 (segment (start 146.85 101.289862) (end 147.860138 102.3) (width 0.2) (layer "F.Cu") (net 22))
 (segment (start 144.75 97.35) (end 144.75 99.245) (width 0.2) (layer "F.Cu") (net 22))
 (segment (start 146.995 99.4) (end 147.075 99.32) (width 0.2) (layer "F.Cu") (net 22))
 (segment (start 146.85 101.289862) (end 146.85 99.45) (width 0.2) (layer "F.Cu") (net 22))
 (segment (start 145.25 97.1) (end 145 97.1) (width 0.2) (layer "F.Cu") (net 22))
 (segment (start 145.55 96.8) (end 145.25 97.1) (width 0.2) (layer "F.Cu") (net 22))
 (segment (start 144.75 99.245) (end 144.905 99.4) (width 0.2) (layer "F.Cu") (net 22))
 (segment (start 147.860138 102.3) (end 148.375 102.3) (width 0.2) (layer "F.Cu") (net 22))
 (segment (start 147.075 99.32) (end 147.075 97.85) (width 0.2) (layer "F.Cu") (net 22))
 (segment (start 147.075 97.825) (end 147.72 97.18) (width 0.2) (layer "F.Cu") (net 22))
 (segment (start 144.8 95.7) (end 145.15 95.7) (width 0.2) (layer "F.Cu") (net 22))
 (segment (start 145.9 100.05) (end 145.715 99.865) (width 0.2) (layer "F.Cu") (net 23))
 (segment (start 148.375 102.7) (end 147.765164 102.7) (width 0.2) (layer "F.Cu") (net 23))
 (segment (start 144.835 99.865) (end 144.4 99.43) (width 0.2) (layer "F.Cu") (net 23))
 (segment (start 145.715 99.865) (end 144.835 99.865) (width 0.2) (layer "F.Cu") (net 23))
 (segment (start 144.4 96.9) (end 144.8 96.5) (width 0.2) (layer "F.Cu") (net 23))
 (segment (start 146.36 100.93) (end 145.9 100.93) (width 0.2) (layer "F.Cu") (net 23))
 (segment (start 145.9 100.93) (end 145.9 100.05) (width 0.2) (layer "F.Cu") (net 23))
 (segment (start 147.765164 102.7) (end 146.48 101.414836) (width 0.2) (layer "F.Cu") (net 23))
 (segment (start 144.82 96.52) (end 144.8 96.5) (width 0.2) (layer "F.Cu") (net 23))
 (segment (start 146.48 101.05) (end 146.36 100.93) (width 0.2) (layer "F.Cu") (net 23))
 (segment (start 146.48 101.414836) (end 146.48 101.05) (width 0.2) (layer "F.Cu") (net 23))
 (segment (start 144.4 99.43) (end 144.4 96.9) (width 0.2) (layer "F.Cu") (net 23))
 (segment (start 151.4375 95.15) (end 150.7325 94.445) (width 0.4) (layer "F.Cu") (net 1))
 (segment (start 150.7325 94.445) (end 150.7325 93.9) (width 0.4) (layer "F.Cu") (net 1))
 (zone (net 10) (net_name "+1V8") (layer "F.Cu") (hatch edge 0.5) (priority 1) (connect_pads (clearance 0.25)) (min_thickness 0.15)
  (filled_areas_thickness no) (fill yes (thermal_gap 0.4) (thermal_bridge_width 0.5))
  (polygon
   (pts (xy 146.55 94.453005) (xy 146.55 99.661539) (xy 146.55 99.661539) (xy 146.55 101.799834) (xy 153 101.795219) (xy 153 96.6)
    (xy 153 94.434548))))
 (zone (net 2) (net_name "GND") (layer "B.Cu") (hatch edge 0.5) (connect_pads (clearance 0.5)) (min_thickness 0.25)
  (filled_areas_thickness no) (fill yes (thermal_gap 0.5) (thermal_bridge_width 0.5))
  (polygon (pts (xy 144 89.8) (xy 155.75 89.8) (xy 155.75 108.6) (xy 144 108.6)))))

